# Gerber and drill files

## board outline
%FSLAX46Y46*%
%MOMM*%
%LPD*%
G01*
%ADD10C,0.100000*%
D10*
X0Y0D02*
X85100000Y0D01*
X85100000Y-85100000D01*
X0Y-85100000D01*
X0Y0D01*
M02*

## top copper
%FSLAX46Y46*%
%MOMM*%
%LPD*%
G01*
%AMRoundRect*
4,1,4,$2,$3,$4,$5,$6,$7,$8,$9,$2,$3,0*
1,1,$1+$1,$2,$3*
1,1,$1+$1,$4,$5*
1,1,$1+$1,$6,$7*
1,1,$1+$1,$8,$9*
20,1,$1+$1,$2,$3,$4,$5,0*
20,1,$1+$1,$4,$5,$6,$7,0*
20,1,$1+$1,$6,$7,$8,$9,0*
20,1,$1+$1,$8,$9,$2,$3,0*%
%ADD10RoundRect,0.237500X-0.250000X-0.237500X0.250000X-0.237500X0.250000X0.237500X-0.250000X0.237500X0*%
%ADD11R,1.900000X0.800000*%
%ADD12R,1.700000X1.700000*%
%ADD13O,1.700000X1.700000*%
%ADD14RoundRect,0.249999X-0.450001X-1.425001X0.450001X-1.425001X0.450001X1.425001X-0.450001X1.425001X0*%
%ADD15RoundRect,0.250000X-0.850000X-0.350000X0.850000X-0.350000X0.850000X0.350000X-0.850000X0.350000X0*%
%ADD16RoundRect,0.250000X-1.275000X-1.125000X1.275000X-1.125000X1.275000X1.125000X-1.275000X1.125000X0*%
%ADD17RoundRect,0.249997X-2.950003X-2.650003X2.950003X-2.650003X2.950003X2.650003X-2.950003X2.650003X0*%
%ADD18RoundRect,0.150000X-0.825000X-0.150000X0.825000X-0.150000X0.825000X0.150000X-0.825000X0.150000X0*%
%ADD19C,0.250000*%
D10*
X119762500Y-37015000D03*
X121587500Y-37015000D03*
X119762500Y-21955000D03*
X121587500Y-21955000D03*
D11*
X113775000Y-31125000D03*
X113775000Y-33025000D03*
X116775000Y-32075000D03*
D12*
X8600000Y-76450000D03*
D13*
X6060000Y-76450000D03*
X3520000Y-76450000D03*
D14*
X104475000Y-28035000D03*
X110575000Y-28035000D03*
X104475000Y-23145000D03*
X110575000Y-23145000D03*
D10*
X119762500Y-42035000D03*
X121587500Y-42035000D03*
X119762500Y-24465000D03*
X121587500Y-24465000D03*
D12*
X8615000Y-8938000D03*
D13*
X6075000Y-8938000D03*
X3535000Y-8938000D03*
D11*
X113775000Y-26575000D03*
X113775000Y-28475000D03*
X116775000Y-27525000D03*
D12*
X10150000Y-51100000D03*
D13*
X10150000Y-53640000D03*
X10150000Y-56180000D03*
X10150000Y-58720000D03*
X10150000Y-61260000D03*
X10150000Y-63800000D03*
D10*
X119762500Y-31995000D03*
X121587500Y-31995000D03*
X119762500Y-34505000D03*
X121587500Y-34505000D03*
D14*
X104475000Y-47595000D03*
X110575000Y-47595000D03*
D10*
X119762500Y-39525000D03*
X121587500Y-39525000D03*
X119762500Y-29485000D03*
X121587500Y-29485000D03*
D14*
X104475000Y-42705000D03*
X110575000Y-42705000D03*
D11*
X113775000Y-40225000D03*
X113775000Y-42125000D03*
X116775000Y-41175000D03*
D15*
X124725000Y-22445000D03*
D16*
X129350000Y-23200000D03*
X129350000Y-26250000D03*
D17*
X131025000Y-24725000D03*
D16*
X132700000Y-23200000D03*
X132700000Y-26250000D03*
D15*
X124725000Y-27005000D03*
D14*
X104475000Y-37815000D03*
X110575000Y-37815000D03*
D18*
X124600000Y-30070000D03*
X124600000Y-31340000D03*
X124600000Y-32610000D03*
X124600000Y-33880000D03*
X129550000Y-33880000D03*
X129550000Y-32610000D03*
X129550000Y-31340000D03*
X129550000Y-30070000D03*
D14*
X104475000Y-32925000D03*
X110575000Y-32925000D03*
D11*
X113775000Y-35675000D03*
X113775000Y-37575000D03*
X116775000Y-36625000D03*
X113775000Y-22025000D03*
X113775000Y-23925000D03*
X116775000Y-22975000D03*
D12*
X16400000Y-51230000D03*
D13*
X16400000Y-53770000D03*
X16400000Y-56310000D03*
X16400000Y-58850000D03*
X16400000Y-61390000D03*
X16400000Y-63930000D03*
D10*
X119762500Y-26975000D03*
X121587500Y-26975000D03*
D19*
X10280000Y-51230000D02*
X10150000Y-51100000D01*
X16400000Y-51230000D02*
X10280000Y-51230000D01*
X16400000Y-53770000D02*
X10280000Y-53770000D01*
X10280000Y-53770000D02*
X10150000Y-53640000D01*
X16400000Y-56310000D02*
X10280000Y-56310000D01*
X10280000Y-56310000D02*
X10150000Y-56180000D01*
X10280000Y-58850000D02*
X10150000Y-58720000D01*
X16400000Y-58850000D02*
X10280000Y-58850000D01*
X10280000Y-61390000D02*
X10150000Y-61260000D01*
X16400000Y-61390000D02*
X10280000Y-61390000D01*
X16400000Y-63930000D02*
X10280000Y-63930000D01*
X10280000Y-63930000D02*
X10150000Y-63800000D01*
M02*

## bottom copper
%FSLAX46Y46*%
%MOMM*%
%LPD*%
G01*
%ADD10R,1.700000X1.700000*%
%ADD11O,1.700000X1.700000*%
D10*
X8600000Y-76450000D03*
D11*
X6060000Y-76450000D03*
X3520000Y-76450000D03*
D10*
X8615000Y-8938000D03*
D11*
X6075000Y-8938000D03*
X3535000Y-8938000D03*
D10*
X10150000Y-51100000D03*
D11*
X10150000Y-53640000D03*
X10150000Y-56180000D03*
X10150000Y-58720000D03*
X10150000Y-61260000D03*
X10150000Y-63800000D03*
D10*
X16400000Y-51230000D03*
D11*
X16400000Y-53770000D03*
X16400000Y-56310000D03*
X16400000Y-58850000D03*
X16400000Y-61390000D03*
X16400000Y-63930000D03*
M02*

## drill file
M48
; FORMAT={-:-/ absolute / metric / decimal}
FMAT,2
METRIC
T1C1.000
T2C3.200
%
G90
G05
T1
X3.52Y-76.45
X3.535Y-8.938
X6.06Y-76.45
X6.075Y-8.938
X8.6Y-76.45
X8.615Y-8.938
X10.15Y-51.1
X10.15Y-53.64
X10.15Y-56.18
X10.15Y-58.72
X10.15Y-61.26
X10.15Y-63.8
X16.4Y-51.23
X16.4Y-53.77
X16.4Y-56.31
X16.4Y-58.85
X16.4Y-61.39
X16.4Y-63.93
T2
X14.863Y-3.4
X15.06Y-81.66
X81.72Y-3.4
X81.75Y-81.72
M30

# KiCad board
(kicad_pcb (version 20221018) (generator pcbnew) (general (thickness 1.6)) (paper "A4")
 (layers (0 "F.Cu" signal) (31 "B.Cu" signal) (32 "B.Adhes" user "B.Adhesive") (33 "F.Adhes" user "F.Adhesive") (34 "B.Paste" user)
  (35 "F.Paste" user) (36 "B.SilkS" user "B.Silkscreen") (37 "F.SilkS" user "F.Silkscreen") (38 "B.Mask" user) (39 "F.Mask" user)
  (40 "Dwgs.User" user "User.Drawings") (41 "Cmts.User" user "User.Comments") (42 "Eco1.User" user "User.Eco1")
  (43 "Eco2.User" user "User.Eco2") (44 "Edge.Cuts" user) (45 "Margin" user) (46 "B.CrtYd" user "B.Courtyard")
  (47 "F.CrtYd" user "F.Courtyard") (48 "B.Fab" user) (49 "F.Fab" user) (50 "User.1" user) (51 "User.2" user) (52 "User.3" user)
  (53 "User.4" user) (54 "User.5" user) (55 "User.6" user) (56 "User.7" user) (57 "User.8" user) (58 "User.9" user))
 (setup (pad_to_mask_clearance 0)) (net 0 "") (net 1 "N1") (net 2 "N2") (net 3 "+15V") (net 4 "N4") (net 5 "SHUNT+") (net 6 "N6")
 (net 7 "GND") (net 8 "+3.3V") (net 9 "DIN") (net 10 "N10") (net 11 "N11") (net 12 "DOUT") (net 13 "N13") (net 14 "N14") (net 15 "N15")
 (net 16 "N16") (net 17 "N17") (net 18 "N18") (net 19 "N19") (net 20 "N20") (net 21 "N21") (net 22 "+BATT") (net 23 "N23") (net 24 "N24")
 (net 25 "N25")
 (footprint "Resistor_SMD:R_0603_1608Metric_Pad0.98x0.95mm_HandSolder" (layer "F.Cu") (at 120.675 37.015)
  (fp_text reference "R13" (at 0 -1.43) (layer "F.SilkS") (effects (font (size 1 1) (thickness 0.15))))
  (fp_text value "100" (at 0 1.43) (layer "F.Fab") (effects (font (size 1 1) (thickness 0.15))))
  (pad "1" smd roundrect (at -0.9125 0) (size 0.975 0.95) (layers "F.Cu" "F.Paste" "F.Mask") (roundrect_rratio 0.25) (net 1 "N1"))
  (pad "2" smd roundrect (at 0.9125 0) (size 0.975 0.95) (layers "F.Cu" "F.Paste" "F.Mask") (roundrect_rratio 0.25) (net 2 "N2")))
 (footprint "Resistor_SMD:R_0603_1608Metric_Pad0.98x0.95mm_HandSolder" (layer "F.Cu") (at 120.675 21.955)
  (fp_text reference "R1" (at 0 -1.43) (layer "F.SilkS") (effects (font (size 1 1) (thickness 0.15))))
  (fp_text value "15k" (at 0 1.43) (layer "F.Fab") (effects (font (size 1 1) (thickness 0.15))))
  (pad "1" smd roundrect (at -0.9125 0) (size 0.975 0.95) (layers "F.Cu" "F.Paste" "F.Mask") (roundrect_rratio 0.25) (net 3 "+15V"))
  (pad "2" smd roundrect (at 0.9125 0) (size 0.975 0.95) (layers "F.Cu" "F.Paste" "F.Mask") (roundrect_rratio 0.25) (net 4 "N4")))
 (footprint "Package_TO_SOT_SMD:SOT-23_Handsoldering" (layer "F.Cu") (at 115.275 32.075)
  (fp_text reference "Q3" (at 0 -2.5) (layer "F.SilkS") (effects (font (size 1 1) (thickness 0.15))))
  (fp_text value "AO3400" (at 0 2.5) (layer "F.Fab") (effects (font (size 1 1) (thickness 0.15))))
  (pad "1" smd rect (at -1.5 -0.95) (size 1.9 0.8) (layers "F.Cu" "F.Paste" "F.Mask") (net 1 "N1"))
  (pad "2" smd rect (at -1.5 0.95) (size 1.9 0.8) (layers "F.Cu" "F.Paste" "F.Mask") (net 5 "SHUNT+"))
  (pad "3" smd rect (at 1.5 0) (size 1.9 0.8) (layers "F.Cu" "F.Paste" "F.Mask") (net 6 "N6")))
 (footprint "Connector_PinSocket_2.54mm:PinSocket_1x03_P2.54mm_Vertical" (layer "F.Cu") (at 8.6 76.45 -90)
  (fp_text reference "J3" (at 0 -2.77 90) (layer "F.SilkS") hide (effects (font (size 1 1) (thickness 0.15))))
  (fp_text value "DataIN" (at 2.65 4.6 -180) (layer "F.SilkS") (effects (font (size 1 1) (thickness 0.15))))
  (pad "1" thru_hole rect (at 0 0 270) (size 1.7 1.7) (drill 1) (layers "*.Cu" "*.Mask") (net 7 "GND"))
  (pad "2" thru_hole oval (at 0 2.54 270) (size 1.7 1.7) (drill 1) (layers "*.Cu" "*.Mask") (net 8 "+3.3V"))
  (pad "3" thru_hole oval (at 0 5.08 270) (size 1.7 1.7) (drill 1) (layers "*.Cu" "*.Mask") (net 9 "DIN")))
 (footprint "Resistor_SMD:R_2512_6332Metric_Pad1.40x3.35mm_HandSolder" (layer "F.Cu") (at 107.525 28.035)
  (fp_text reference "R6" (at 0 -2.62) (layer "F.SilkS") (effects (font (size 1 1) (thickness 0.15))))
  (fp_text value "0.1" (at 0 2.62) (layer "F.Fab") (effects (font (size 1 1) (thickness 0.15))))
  (pad "1" smd roundrect (at -3.05 0) (size 1.4 3.35) (layers "F.Cu" "F.Paste" "F.Mask") (roundrect_rratio 0.178571) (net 7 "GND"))
  (pad "2" smd roundrect (at 3.05 0) (size 1.4 3.35) (layers "F.Cu" "F.Paste" "F.Mask") (roundrect_rratio 0.178571) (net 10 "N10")))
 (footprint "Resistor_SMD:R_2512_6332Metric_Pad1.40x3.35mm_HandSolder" (layer "F.Cu") (at 107.525 23.145)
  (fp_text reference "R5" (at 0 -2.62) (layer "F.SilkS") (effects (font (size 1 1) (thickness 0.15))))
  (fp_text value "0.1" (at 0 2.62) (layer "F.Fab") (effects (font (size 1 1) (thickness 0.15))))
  (pad "1" smd roundrect (at -3.05 0) (size 1.4 3.35) (layers "F.Cu" "F.Paste" "F.Mask") (roundrect_rratio 0.178571) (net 7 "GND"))
  (pad "2" smd roundrect (at 3.05 0) (size 1.4 3.35) (layers "F.Cu" "F.Paste" "F.Mask") (roundrect_rratio 0.178571) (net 10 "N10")))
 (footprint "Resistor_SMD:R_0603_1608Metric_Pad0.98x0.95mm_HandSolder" (layer "F.Cu") (at 120.675 42.035)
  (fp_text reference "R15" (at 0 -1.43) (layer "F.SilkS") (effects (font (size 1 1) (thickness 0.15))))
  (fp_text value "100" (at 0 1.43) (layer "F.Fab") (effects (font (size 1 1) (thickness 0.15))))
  (pad "1" smd roundrect (at -0.9125 0) (size 0.975 0.95) (layers "F.Cu" "F.Paste" "F.Mask") (roundrect_rratio 0.25) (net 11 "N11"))
  (pad "2" smd roundrect (at 0.9125 0) (size 0.975 0.95) (layers "F.Cu" "F.Paste" "F.Mask") (roundrect_rratio 0.25) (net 2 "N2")))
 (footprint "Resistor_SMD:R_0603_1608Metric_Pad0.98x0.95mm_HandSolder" (layer "F.Cu") (at 120.675 24.465)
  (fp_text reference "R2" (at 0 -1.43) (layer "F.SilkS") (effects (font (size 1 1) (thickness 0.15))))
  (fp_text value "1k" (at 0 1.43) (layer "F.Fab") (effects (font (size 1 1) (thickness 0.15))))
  (pad "1" smd roundrect (at -0.9125 0) (size 0.975 0.95) (layers "F.Cu" "F.Paste" "F.Mask") (roundrect_rratio 0.25) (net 7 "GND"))
  (pad "2" smd roundrect (at 0.9125 0) (size 0.975 0.95) (layers "F.Cu" "F.Paste" "F.Mask") (roundrect_rratio 0.25) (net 4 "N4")))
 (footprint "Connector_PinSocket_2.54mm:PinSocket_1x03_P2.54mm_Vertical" (layer "F.Cu") (at 8.615 8.938 -90)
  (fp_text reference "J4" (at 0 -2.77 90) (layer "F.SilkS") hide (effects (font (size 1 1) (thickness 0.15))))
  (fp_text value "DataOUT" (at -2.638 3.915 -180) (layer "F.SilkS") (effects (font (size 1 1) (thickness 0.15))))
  (pad "1" thru_hole rect (at 0 0 270) (size 1.7 1.7) (drill 1) (layers "*.Cu" "*.Mask") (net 7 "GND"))
  (pad "2" thru_hole oval (at 0 2.54 270) (size 1.7 1.7) (drill 1) (layers "*.Cu" "*.Mask") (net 8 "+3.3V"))
  (pad "3" thru_hole oval (at 0 5.08 270) (size 1.7 1.7) (drill 1) (layers "*.Cu" "*.Mask") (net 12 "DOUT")))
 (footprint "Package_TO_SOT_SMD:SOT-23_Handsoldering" (layer "F.Cu") (at 115.275 27.525)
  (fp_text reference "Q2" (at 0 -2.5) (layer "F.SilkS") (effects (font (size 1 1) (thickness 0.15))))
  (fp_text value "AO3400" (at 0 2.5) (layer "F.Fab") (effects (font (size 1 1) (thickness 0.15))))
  (pad "1" smd rect (at -1.5 -0.95) (size 1.9 0.8) (layers "F.Cu" "F.Paste" "F.Mask") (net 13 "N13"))
  (pad "2" smd rect (at -1.5 0.95) (size 1.9 0.8) (layers "F.Cu" "F.Paste" "F.Mask") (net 5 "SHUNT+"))
  (pad "3" smd rect (at 1.5 0) (size 1.9 0.8) (layers "F.Cu" "F.Paste" "F.Mask") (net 6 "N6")))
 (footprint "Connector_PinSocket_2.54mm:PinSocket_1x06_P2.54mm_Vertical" (layer "F.Cu") (at 10.15 51.1)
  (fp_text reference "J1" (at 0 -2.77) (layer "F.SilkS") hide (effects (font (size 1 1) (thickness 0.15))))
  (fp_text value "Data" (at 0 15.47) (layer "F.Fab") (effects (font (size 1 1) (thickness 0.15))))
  (pad "1" thru_hole rect (at 0 0) (size 1.7 1.7) (drill 1) (layers "*.Cu" "*.Mask") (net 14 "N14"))
  (pad "2" thru_hole oval (at 0 2.54) (size 1.7 1.7) (drill 1) (layers "*.Cu" "*.Mask") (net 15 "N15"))
  (pad "3" thru_hole oval (at 0 5.08) (size 1.7 1.7) (drill 1) (layers "*.Cu" "*.Mask") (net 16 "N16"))
  (pad "4" thru_hole oval (at 0 7.62) (size 1.7 1.7) (drill 1) (layers "*.Cu" "*.Mask") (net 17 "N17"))
  (pad "5" thru_hole oval (at 0 10.16) (size 1.7 1.7) (drill 1) (layers "*.Cu" "*.Mask") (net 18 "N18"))
  (pad "6" thru_hole oval (at 0 12.7) (size 1.7 1.7) (drill 1) (layers "*.Cu" "*.Mask") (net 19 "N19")))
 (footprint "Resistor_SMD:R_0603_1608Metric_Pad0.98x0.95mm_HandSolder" (layer "F.Cu") (at 120.675 31.995)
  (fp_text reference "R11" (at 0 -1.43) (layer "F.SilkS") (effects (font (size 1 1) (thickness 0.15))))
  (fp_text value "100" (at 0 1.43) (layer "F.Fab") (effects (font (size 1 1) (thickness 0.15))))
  (pad "1" smd roundrect (at -0.9125 0) (size 0.975 0.95) (layers "F.Cu" "F.Paste" "F.Mask") (roundrect_rratio 0.25) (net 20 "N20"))
  (pad "2" smd roundrect (at 0.9125 0) (size 0.975 0.95) (layers "F.Cu" "F.Paste" "F.Mask") (roundrect_rratio 0.25) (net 2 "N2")))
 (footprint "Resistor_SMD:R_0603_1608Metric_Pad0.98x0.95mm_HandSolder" (layer "F.Cu") (at 120.675 34.505)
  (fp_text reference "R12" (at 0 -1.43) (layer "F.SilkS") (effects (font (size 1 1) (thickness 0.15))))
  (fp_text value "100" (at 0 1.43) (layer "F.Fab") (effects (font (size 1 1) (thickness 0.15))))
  (pad "1" smd roundrect (at -0.9125 0) (size 0.975 0.95) (layers "F.Cu" "F.Paste" "F.Mask") (roundrect_rratio 0.25) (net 13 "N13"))
  (pad "2" smd roundrect (at 0.9125 0) (size 0.975 0.95) (layers "F.Cu" "F.Paste" "F.Mask") (roundrect_rratio 0.25) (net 2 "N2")))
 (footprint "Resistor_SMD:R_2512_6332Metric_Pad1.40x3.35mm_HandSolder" (layer "F.Cu") (at 107.525 47.595)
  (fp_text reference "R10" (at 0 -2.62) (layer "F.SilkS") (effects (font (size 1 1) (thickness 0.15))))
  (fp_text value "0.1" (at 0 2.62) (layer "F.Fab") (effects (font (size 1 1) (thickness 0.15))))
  (pad "1" smd roundrect (at -3.05 0) (size 1.4 3.35) (layers "F.Cu" "F.Paste" "F.Mask") (roundrect_rratio 0.178571) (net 10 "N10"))
  (pad "2" smd roundrect (at 3.05 0) (size 1.4 3.35) (layers "F.Cu" "F.Paste" "F.Mask") (roundrect_rratio 0.178571) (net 5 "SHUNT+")))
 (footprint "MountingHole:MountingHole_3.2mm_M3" (layer "F.Cu") (at 14.863 3.4)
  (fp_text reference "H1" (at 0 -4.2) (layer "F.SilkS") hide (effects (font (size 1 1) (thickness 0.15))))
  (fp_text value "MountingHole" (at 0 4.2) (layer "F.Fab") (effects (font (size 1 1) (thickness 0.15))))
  (pad "" np_thru_hole circle (at 0 0) (size 3.2 3.2) (drill 3.2) (layers "*.Cu" "*.Mask")))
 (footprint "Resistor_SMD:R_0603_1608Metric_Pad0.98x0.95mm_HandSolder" (layer "F.Cu") (at 120.675 39.525)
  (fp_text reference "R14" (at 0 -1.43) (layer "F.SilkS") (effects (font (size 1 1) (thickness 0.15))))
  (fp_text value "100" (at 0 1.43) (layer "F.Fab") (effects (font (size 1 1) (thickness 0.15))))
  (pad "1" smd roundrect (at -0.9125 0) (size 0.975 0.95) (layers "F.Cu" "F.Paste" "F.Mask") (roundrect_rratio 0.25) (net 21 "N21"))
  (pad "2" smd roundrect (at 0.9125 0) (size 0.975 0.95) (layers "F.Cu" "F.Paste" "F.Mask") (roundrect_rratio 0.25) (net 2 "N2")))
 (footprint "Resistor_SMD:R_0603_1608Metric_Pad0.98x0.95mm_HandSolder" (layer "F.Cu") (at 120.675 29.485)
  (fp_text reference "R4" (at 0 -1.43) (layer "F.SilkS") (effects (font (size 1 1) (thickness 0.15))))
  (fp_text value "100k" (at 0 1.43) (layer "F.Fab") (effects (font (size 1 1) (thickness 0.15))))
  (pad "1" smd roundrect (at -0.9125 0) (size 0.975 0.95) (layers "F.Cu" "F.Paste" "F.Mask") (roundrect_rratio 0.25) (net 2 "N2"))
  (pad "2" smd roundrect (at 0.9125 0) (size 0.975 0.95) (layers "F.Cu" "F.Paste" "F.Mask") (roundrect_rratio 0.25) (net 3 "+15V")))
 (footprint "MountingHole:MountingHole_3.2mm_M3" (layer "F.Cu") (at 15.06 81.66)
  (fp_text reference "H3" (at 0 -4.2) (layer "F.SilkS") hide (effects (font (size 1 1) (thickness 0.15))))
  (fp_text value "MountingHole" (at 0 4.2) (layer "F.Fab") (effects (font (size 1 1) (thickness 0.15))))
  (pad "" np_thru_hole circle (at 0 0) (size 3.2 3.2) (drill 3.2) (layers "*.Cu" "*.Mask")))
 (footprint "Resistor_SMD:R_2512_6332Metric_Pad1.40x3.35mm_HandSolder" (layer "F.Cu") (at 107.525 42.705)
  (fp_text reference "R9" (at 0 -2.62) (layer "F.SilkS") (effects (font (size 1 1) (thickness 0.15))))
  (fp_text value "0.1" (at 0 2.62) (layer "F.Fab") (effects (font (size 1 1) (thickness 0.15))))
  (pad "1" smd roundrect (at -3.05 0) (size 1.4 3.35) (layers "F.Cu" "F.Paste" "F.Mask") (roundrect_rratio 0.178571) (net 10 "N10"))
  (pad "2" smd roundrect (at 3.05 0) (size 1.4 3.35) (layers "F.Cu" "F.Paste" "F.Mask") (roundrect_rratio 0.178571) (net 5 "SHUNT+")))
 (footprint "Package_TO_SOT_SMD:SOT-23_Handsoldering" (layer "F.Cu") (at 115.275 41.175)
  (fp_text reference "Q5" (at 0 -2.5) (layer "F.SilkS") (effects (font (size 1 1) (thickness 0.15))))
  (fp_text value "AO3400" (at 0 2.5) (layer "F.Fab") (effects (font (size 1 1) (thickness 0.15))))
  (pad "1" smd rect (at -1.5 -0.95) (size 1.9 0.8) (layers "F.Cu" "F.Paste" "F.Mask") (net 11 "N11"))
  (pad "2" smd rect (at -1.5 0.95) (size 1.9 0.8) (layers "F.Cu" "F.Paste" "F.Mask") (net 5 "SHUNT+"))
  (pad "3" smd rect (at 1.5 0) (size 1.9 0.8) (layers "F.Cu" "F.Paste" "F.Mask") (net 6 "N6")))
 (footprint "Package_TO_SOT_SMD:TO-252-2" (layer "F.Cu") (at 129.765 24.725)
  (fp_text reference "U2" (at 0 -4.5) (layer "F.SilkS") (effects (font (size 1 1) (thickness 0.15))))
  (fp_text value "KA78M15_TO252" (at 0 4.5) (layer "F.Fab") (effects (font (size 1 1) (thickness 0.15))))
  (pad "1" smd roundrect (at -5.04 -2.28) (size 2.2 1.2) (layers "F.Cu" "F.Paste" "F.Mask") (roundrect_rratio 0.208333) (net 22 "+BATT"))
  (pad "2" smd roundrect (at -0.415 -1.525) (size 3.05 2.75) (layers "F.Cu" "F.Paste") (roundrect_rratio 0.090909) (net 7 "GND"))
  (pad "2" smd roundrect (at -0.415 1.525) (size 3.05 2.75) (layers "F.Cu" "F.Paste") (roundrect_rratio 0.090909) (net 7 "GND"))
  (pad "2" smd roundrect (at 1.26 0) (size 6.4 5.8) (layers "F.Cu" "F.Mask") (roundrect_rratio 0.043103) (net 7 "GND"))
  (pad "2" smd roundrect (at 2.935 -1.525) (size 3.05 2.75) (layers "F.Cu" "F.Paste") (roundrect_rratio 0.090909) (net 7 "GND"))
  (pad "2" smd roundrect (at 2.935 1.525) (size 3.05 2.75) (layers "F.Cu" "F.Paste") (roundrect_rratio 0.090909) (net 7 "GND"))
  (pad "3" smd roundrect (at -5.04 2.28) (size 2.2 1.2) (layers "F.Cu" "F.Paste" "F.Mask") (roundrect_rratio 0.208333) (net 3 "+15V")))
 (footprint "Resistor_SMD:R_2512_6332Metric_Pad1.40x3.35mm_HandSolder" (layer "F.Cu") (at 107.525 37.815)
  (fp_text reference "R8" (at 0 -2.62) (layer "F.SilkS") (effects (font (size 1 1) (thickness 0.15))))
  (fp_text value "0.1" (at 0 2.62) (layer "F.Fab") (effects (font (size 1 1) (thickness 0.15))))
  (pad "1" smd roundrect (at -3.05 0) (size 1.4 3.35) (layers "F.Cu" "F.Paste" "F.Mask") (roundrect_rratio 0.178571) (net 10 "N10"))
  (pad "2" smd roundrect (at 3.05 0) (size 1.4 3.35) (layers "F.Cu" "F.Paste" "F.Mask") (roundrect_rratio 0.178571) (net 5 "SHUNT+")))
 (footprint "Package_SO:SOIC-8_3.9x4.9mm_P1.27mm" (layer "F.Cu") (at 127.075 31.975)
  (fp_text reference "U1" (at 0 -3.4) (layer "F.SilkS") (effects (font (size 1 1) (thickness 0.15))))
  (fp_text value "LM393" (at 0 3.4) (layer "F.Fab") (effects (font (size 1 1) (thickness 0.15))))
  (pad "1" smd roundrect (at -2.475 -1.905) (size 1.95 0.6) (layers "F.Cu" "F.Paste" "F.Mask") (roundrect_rratio 0.25) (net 2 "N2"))
  (pad "2" smd roundrect (at -2.475 -0.635) (size 1.95 0.6) (layers "F.Cu" "F.Paste" "F.Mask") (roundrect_rratio 0.25) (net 5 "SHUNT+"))
  (pad "3" smd roundrect (at -2.475 0.635) (size 1.95 0.6) (layers "F.Cu" "F.Paste" "F.Mask") (roundrect_rratio 0.25) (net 4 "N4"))
  (pad "4" smd roundrect (at -2.475 1.905) (size 1.95 0.6) (layers "F.Cu" "F.Paste" "F.Mask") (roundrect_rratio 0.25) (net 7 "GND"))
  (pad "5" smd roundrect (at 2.475 1.905) (size 1.95 0.6) (layers "F.Cu" "F.Paste" "F.Mask") (roundrect_rratio 0.25) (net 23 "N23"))
  (pad "6" smd roundrect (at 2.475 0.635) (size 1.95 0.6) (layers "F.Cu" "F.Paste" "F.Mask") (roundrect_rratio 0.25) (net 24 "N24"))
  (pad "7" smd roundrect (at 2.475 -0.635) (size 1.95 0.6) (layers "F.Cu" "F.Paste" "F.Mask") (roundrect_rratio 0.25) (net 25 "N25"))
  (pad "8" smd roundrect (at 2.475 -1.905) (size 1.95 0.6) (layers "F.Cu" "F.Paste" "F.Mask") (roundrect_rratio 0.25) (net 3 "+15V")))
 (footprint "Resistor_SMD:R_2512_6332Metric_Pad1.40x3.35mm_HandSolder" (layer "F.Cu") (at 107.525 32.925)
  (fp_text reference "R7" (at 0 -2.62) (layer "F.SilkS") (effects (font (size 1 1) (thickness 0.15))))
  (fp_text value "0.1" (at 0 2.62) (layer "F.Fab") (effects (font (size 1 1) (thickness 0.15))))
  (pad "1" smd roundrect (at -3.05 0) (size 1.4 3.35) (layers "F.Cu" "F.Paste" "F.Mask") (roundrect_rratio 0.178571) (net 7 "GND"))
  (pad "2" smd roundrect (at 3.05 0) (size 1.4 3.35) (layers "F.Cu" "F.Paste" "F.Mask") (roundrect_rratio 0.178571) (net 10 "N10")))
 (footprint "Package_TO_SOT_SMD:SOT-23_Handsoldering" (layer "F.Cu") (at 115.275 36.625)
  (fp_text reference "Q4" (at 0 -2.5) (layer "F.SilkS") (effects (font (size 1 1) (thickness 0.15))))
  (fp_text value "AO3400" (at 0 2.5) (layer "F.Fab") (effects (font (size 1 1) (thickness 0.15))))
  (pad "1" smd rect (at -1.5 -0.95) (size 1.9 0.8) (layers "F.Cu" "F.Paste" "F.Mask") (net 21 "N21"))
  (pad "2" smd rect (at -1.5 0.95) (size 1.9 0.8) (layers "F.Cu" "F.Paste" "F.Mask") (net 5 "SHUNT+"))
  (pad "3" smd rect (at 1.5 0) (size 1.9 0.8) (layers "F.Cu" "F.Paste" "F.Mask") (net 6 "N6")))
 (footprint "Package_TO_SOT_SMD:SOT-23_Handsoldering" (layer "F.Cu") (at 115.275 22.975)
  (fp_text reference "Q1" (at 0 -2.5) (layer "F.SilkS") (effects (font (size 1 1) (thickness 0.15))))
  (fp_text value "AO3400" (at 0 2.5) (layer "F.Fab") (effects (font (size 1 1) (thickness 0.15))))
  (pad "1" smd rect (at -1.5 -0.95) (size 1.9 0.8) (layers "F.Cu" "F.Paste" "F.Mask") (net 20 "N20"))
  (pad "2" smd rect (at -1.5 0.95) (size 1.9 0.8) (layers "F.Cu" "F.Paste" "F.Mask") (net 5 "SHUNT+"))
  (pad "3" smd rect (at 1.5 0) (size 1.9 0.8) (layers "F.Cu" "F.Paste" "F.Mask") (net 6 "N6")))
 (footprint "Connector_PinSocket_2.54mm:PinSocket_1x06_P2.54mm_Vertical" (layer "F.Cu") (at 16.4 51.23)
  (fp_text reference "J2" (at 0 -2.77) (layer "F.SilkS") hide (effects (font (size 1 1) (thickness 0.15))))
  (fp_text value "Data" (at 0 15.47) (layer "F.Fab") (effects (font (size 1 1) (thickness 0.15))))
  (pad "1" thru_hole rect (at 0 0) (size 1.7 1.7) (drill 1) (layers "*.Cu" "*.Mask") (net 14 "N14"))
  (pad "2" thru_hole oval (at 0 2.54) (size 1.7 1.7) (drill 1) (layers "*.Cu" "*.Mask") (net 15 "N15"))
  (pad "3" thru_hole oval (at 0 5.08) (size 1.7 1.7) (drill 1) (layers "*.Cu" "*.Mask") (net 16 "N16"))
  (pad "4" thru_hole oval (at 0 7.62) (size 1.7 1.7) (drill 1) (layers "*.Cu" "*.Mask") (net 17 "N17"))
  (pad "5" thru_hole oval (at 0 10.16) (size 1.7 1.7) (drill 1) (layers "*.Cu" "*.Mask") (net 18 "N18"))
  (pad "6" thru_hole oval (at 0 12.7) (size 1.7 1.7) (drill 1) (layers "*.Cu" "*.Mask") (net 19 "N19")))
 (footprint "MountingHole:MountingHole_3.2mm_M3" (layer "F.Cu") (at 81.75 81.72)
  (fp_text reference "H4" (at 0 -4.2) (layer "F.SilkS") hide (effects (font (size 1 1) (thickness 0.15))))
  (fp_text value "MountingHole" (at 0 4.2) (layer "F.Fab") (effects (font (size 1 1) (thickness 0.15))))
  (pad "" np_thru_hole circle (at 0 0) (size 3.2 3.2) (drill 3.2) (layers "*.Cu" "*.Mask")))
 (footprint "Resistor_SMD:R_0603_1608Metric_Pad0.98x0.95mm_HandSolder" (layer "F.Cu") (at 120.675 26.975)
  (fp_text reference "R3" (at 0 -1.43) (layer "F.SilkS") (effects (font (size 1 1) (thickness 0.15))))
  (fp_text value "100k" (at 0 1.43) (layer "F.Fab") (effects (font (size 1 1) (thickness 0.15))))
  (pad "1" smd roundrect (at -0.9125 0) (size 0.975 0.95) (layers "F.Cu" "F.Paste" "F.Mask") (roundrect_rratio 0.25) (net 7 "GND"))
  (pad "2" smd roundrect (at 0.9125 0) (size 0.975 0.95) (layers "F.Cu" "F.Paste" "F.Mask") (roundrect_rratio 0.25) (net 2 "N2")))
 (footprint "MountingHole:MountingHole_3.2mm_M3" (layer "F.Cu") (at 81.72 3.4)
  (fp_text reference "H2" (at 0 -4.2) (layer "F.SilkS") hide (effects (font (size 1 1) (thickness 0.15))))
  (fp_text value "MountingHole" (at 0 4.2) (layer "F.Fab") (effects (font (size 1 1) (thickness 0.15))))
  (pad "" np_thru_hole circle (at 0 0) (size 3.2 3.2) (drill 3.2) (layers "*.Cu" "*.Mask")))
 (gr_rect (start 0 0) (end 85.1 85.1) (stroke (width 0.1) (type default)) (fill none) (layer "Edge.Cuts"))
 (segment (start 10.28 51.23) (end 10.15 51.1) (width 0.25) (layer "F.Cu") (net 14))
 (segment (start 16.4 51.23) (end 10.28 51.23) (width 0.25) (layer "F.Cu") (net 14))
 (segment (start 16.4 53.77) (end 10.28 53.77) (width 0.25) (layer "F.Cu") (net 15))
 (segment (start 10.28 53.77) (end 10.15 53.64) (width 0.25) (layer "F.Cu") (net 15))
 (segment (start 16.4 56.31) (end 10.28 56.31) (width 0.25) (layer "F.Cu") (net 16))
 (segment (start 10.28 56.31) (end 10.15 56.18) (width 0.25) (layer "F.Cu") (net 16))
 (segment (start 10.28 58.85) (end 10.15 58.72) (width 0.25) (layer "F.Cu") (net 17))
 (segment (start 16.4 58.85) (end 10.28 58.85) (width 0.25) (layer "F.Cu") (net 17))
 (segment (start 10.28 61.39) (end 10.15 61.26) (width 0.25) (layer "F.Cu") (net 18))
 (segment (start 16.4 61.39) (end 10.28 61.39) (width 0.25) (layer "F.Cu") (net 18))
 (segment (start 16.4 63.93) (end 10.28 63.93) (width 0.25) (layer "F.Cu") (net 19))
 (segment (start 10.28 63.93) (end 10.15 63.8) (width 0.25) (layer "F.Cu") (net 19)))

